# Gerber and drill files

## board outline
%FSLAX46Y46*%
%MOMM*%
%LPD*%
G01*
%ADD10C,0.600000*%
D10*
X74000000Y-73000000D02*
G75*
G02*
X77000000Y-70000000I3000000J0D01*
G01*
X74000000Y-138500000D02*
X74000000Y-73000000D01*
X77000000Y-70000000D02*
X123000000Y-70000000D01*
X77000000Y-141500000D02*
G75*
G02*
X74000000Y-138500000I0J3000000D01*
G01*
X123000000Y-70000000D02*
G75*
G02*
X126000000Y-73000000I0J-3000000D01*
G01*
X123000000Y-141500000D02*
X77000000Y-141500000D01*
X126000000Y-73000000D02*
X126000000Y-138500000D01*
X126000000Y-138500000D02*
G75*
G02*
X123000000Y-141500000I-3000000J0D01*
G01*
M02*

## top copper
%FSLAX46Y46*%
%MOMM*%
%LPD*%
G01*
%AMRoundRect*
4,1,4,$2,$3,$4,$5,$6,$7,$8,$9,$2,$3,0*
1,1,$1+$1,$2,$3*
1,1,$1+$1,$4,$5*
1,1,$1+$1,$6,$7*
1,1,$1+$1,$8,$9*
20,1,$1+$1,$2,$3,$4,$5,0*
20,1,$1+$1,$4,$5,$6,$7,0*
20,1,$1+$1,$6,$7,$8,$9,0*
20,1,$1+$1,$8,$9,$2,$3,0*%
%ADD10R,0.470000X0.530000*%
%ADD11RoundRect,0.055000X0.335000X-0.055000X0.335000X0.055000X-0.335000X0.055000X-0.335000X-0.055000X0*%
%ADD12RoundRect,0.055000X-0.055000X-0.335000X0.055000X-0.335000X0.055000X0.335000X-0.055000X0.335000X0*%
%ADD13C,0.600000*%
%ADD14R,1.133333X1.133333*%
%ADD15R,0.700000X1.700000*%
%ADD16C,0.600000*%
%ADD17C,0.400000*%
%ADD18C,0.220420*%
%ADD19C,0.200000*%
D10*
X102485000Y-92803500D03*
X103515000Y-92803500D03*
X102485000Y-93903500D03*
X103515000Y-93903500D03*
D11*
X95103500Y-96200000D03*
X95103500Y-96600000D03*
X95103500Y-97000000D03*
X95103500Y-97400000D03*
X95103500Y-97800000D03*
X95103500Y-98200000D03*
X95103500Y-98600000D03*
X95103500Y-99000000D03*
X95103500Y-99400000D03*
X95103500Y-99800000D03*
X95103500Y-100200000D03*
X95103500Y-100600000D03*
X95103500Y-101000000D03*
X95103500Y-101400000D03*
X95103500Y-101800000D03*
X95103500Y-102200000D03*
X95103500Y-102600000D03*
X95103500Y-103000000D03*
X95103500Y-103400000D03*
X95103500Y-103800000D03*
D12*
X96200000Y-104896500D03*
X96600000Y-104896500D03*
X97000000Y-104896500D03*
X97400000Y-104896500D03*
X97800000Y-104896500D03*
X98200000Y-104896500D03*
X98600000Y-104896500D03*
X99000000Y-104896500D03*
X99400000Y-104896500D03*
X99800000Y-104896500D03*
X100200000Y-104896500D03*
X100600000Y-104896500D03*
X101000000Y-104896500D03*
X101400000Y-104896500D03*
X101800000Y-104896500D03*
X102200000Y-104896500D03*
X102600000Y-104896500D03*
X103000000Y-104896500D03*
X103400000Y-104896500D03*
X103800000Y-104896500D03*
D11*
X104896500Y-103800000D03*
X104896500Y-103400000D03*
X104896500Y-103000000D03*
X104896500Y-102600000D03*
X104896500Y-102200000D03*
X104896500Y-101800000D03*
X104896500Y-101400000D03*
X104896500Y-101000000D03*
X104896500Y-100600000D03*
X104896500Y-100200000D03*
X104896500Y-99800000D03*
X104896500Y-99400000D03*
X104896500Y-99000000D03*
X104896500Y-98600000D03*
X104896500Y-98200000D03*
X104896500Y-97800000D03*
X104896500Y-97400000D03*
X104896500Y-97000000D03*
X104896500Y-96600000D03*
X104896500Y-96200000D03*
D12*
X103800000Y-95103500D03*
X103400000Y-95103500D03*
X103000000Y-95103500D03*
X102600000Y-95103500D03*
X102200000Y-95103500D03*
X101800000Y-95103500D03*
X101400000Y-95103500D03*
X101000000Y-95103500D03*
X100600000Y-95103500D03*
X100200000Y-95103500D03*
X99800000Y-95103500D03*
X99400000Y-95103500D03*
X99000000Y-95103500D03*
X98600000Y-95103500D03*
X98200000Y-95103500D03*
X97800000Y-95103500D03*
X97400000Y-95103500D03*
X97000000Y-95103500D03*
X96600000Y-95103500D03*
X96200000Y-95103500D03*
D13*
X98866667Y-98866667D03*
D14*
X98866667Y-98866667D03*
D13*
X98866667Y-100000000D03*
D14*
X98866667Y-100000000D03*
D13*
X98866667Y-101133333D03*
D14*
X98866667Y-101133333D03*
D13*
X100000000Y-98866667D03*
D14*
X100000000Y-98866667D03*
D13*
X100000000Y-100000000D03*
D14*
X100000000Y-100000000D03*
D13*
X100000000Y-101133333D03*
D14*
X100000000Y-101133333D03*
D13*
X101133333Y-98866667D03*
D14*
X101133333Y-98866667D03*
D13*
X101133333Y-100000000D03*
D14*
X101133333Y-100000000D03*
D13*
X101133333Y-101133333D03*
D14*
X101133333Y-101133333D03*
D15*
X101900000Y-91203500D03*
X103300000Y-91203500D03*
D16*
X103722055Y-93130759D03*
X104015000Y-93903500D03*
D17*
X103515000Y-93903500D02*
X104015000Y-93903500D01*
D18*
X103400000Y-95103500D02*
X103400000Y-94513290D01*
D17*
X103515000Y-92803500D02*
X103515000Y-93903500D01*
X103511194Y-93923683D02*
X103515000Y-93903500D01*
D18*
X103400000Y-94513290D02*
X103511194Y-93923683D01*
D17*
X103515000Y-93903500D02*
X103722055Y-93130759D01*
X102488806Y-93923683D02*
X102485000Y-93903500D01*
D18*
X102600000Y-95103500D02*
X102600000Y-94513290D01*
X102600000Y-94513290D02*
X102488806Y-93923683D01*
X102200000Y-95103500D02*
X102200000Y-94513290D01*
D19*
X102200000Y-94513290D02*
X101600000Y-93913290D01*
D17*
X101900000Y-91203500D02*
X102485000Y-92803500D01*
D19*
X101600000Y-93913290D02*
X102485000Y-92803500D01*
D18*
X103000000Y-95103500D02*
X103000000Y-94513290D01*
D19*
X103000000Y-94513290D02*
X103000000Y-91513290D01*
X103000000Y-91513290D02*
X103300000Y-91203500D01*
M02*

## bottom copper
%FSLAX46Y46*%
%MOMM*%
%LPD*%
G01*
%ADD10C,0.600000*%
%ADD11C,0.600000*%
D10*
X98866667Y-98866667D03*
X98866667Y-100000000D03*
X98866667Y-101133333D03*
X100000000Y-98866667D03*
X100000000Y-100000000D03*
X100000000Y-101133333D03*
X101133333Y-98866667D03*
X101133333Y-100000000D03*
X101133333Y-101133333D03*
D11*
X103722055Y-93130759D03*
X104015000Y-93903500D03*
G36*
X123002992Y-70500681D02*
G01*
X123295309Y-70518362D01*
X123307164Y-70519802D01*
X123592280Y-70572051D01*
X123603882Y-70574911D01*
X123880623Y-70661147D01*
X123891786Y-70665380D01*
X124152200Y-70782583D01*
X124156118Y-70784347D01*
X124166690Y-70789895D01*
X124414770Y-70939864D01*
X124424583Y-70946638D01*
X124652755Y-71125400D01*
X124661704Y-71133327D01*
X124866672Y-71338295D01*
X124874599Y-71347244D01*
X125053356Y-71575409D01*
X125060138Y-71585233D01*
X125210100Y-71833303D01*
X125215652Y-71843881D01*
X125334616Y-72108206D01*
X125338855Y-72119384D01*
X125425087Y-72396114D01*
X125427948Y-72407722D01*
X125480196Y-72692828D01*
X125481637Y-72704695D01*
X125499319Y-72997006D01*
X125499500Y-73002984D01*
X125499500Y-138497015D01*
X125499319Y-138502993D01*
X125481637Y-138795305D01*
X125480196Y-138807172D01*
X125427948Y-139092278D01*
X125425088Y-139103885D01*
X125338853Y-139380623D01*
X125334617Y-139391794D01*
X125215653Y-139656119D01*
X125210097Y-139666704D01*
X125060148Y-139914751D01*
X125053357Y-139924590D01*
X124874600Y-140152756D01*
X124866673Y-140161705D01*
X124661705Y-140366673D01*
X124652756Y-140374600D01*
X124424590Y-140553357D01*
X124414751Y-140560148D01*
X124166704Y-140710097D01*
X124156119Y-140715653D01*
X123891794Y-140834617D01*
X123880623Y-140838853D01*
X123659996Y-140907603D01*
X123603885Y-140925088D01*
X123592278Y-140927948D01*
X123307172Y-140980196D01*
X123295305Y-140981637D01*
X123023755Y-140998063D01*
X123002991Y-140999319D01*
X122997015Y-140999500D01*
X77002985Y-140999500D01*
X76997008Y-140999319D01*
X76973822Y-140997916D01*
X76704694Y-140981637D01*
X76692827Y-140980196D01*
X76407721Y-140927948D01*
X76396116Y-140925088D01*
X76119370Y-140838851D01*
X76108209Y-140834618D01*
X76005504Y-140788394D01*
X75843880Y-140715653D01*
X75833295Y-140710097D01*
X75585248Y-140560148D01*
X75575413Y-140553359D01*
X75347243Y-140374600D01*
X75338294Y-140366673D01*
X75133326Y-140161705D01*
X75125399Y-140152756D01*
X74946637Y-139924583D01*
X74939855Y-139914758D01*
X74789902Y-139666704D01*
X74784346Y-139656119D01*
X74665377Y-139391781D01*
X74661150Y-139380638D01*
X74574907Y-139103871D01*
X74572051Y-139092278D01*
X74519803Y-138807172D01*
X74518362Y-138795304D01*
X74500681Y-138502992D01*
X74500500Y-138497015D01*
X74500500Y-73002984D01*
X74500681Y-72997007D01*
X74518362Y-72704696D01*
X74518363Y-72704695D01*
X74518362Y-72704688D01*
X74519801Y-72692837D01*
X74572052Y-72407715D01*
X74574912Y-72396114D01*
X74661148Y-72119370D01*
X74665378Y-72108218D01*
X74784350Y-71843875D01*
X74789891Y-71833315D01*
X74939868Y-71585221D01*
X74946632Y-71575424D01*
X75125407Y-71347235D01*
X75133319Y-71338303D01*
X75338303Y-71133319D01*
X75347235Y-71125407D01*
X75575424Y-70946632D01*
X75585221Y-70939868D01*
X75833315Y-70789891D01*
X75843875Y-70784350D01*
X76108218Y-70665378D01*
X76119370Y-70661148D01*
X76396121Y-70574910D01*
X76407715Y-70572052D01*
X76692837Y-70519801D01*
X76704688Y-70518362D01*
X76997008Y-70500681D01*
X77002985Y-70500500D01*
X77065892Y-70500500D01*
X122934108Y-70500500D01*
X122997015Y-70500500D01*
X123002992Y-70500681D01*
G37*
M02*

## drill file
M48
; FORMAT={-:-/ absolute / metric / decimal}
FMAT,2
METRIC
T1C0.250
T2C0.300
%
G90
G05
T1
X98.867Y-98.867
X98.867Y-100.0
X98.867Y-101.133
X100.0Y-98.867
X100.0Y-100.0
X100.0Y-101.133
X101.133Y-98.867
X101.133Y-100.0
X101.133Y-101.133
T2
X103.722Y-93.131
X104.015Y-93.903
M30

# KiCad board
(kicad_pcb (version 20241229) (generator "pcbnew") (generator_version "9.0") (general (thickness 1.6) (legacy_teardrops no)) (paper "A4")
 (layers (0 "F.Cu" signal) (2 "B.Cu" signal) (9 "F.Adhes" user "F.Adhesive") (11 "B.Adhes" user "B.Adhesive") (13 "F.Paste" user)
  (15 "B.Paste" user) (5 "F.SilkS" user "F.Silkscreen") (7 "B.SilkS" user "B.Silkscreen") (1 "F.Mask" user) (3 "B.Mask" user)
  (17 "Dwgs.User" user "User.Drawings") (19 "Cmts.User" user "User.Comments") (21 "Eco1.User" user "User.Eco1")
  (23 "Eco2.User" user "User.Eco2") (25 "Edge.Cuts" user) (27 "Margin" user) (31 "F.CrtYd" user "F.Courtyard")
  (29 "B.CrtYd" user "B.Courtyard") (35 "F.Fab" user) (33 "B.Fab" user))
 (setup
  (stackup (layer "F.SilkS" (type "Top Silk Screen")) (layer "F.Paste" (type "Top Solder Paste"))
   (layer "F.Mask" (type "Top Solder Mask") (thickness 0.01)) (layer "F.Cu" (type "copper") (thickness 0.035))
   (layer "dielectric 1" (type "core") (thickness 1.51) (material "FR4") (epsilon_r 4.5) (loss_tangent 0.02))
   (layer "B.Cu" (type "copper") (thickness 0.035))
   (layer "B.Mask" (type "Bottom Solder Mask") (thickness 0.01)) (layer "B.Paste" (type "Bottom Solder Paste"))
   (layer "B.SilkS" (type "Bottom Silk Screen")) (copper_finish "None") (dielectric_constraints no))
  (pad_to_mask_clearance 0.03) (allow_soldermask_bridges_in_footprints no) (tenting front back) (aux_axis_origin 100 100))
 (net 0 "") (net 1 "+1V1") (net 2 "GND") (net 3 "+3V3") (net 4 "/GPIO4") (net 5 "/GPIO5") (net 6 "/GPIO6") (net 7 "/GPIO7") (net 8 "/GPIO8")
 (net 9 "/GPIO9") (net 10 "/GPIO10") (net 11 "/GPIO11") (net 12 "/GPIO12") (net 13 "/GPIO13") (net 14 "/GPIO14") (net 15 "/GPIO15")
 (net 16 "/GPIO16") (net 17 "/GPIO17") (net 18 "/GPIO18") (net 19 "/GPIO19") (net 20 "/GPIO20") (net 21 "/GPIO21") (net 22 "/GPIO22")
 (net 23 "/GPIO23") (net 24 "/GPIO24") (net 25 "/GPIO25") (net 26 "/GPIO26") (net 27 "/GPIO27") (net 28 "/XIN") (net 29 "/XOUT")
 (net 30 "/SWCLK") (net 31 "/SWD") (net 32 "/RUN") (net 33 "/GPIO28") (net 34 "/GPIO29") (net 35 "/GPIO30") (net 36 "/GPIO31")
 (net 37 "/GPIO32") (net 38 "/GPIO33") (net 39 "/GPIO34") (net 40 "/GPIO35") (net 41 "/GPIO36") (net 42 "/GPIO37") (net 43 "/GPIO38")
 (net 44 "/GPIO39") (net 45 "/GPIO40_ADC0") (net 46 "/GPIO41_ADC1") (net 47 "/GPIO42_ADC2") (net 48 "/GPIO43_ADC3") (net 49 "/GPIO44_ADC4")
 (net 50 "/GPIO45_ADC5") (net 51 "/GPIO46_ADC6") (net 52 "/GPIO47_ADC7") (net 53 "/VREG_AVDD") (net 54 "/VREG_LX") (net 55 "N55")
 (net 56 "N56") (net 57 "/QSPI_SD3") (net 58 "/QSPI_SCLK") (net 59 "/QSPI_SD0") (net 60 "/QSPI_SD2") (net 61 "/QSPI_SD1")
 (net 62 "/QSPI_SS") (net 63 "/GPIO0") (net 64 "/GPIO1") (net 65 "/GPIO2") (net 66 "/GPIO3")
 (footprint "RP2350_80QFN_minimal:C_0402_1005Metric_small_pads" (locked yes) (layer "F.Cu") (at 103 92.8035)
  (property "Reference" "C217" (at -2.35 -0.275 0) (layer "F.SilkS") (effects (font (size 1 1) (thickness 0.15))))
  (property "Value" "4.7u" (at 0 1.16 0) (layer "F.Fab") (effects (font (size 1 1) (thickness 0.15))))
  (pad "1" smd rect (at -0.515 0) (size 0.47 0.53) (layers "F.Cu" "F.Mask" "F.Paste") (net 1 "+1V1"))
  (pad "2" smd rect (at 0.515 0) (size 0.47 0.53) (layers "F.Cu" "F.Mask" "F.Paste") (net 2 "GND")))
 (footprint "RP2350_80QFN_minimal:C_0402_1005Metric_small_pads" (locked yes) (layer "F.Cu") (at 103 93.9035)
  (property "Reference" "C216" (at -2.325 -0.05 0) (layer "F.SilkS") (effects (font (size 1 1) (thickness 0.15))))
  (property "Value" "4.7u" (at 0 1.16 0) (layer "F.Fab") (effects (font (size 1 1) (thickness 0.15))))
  (pad "1" smd rect (at -0.515 0) (size 0.47 0.53) (layers "F.Cu" "F.Mask" "F.Paste") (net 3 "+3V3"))
  (pad "2" smd rect (at 0.515 0) (size 0.47 0.53) (layers "F.Cu" "F.Mask" "F.Paste") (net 2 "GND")))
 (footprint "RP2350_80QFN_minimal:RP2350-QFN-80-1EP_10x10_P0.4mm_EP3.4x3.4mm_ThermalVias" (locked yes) (layer "F.Cu") (at 100 100)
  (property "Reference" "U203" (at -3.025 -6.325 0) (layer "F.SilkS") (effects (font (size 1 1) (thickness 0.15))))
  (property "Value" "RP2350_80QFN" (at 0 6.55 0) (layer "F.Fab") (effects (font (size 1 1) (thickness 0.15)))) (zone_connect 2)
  (pad "" smd roundrect (at -0.7 -0.7) (size 1.2 1.2) (layers "F.Paste") (roundrect_rratio 0.2083333333) (zone_connect 2))
  (pad "" smd roundrect (at -0.7 0.7) (size 1.2 1.2) (layers "F.Paste") (roundrect_rratio 0.2083333333) (zone_connect 2))
  (pad "" smd roundrect (at 0.7 -0.7) (size 1.2 1.2) (layers "F.Paste") (roundrect_rratio 0.2083333333) (zone_connect 2))
  (pad "" smd roundrect (at 0.7 0.7) (size 1.2 1.2) (layers "F.Paste") (roundrect_rratio 0.2083333333) (zone_connect 2))
  (pad "1" smd roundrect (at -4.8965 -3.8 90) (size 0.22 0.78) (layers "F.Cu" "F.Mask" "F.Paste") (roundrect_rratio 0.25) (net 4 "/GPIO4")
   (thermal_bridge_angle 45))
  (pad "2" smd roundrect (at -4.8965 -3.4 90) (size 0.22 0.78) (layers "F.Cu" "F.Mask" "F.Paste") (roundrect_rratio 0.25) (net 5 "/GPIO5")
   (thermal_bridge_angle 45))
  (pad "3" smd roundrect (at -4.8965 -3 90) (size 0.22 0.78) (layers "F.Cu" "F.Mask" "F.Paste") (roundrect_rratio 0.25) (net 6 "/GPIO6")
   (thermal_bridge_angle 45))
  (pad "4" smd roundrect (at -4.8965 -2.6 90) (size 0.22 0.78) (layers "F.Cu" "F.Mask" "F.Paste") (roundrect_rratio 0.25) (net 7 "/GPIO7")
   (thermal_bridge_angle 45))
  (pad "5" smd roundrect (at -4.8965 -2.2 90) (size 0.22 0.78) (layers "F.Cu" "F.Mask" "F.Paste") (roundrect_rratio 0.25) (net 3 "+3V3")
   (thermal_bridge_angle 45))
  (pad "6" smd roundrect (at -4.8965 -1.8 90) (size 0.22 0.78) (layers "F.Cu" "F.Mask" "F.Paste") (roundrect_rratio 0.25) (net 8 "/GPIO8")
   (thermal_bridge_angle 45))
  (pad "7" smd roundrect (at -4.8965 -1.4 90) (size 0.22 0.78) (layers "F.Cu" "F.Mask" "F.Paste") (roundrect_rratio 0.25) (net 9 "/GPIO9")
   (thermal_bridge_angle 45))
  (pad "8" smd roundrect (at -4.8965 -1 90) (size 0.22 0.78) (layers "F.Cu" "F.Mask" "F.Paste") (roundrect_rratio 0.25) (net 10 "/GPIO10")
   (thermal_bridge_angle 45))
  (pad "9" smd roundrect (at -4.8965 -0.6 90) (size 0.22 0.78) (layers "F.Cu" "F.Mask" "F.Paste") (roundrect_rratio 0.25) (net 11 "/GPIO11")
   (thermal_bridge_angle 45))
  (pad "10" smd roundrect (at -4.8965 -0.2 90) (size 0.22 0.78) (layers "F.Cu" "F.Mask" "F.Paste") (roundrect_rratio 0.25) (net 1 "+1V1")
   (thermal_bridge_angle 45))
  (pad "11" smd roundrect (at -4.8965 0.2 90) (size 0.22 0.78) (layers "F.Cu" "F.Mask" "F.Paste") (roundrect_rratio 0.25) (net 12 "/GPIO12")
   (thermal_bridge_angle 45))
  (pad "12" smd roundrect (at -4.8965 0.6 90) (size 0.22 0.78) (layers "F.Cu" "F.Mask" "F.Paste") (roundrect_rratio 0.25) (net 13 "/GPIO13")
   (thermal_bridge_angle 45))
  (pad "13" smd roundrect (at -4.8965 1 90) (size 0.22 0.78) (layers "F.Cu" "F.Mask" "F.Paste") (roundrect_rratio 0.25) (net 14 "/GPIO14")
   (thermal_bridge_angle 45))
  (pad "14" smd roundrect (at -4.8965 1.4 90) (size 0.22 0.78) (layers "F.Cu" "F.Mask" "F.Paste") (roundrect_rratio 0.25) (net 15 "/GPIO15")
   (thermal_bridge_angle 45))
  (pad "15" smd roundrect (at -4.8965 1.8 90) (size 0.22 0.78) (layers "F.Cu" "F.Mask" "F.Paste") (roundrect_rratio 0.25) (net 3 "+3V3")
   (thermal_bridge_angle 45))
  (pad "16" smd roundrect (at -4.8965 2.2 90) (size 0.22 0.78) (layers "F.Cu" "F.Mask" "F.Paste") (roundrect_rratio 0.25) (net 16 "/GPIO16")
   (thermal_bridge_angle 45))
  (pad "17" smd roundrect (at -4.8965 2.6 90) (size 0.22 0.78) (layers "F.Cu" "F.Mask" "F.Paste") (roundrect_rratio 0.25) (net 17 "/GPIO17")
   (thermal_bridge_angle 45))
  (pad "18" smd roundrect (at -4.8965 3 90) (size 0.22 0.78) (layers "F.Cu" "F.Mask" "F.Paste") (roundrect_rratio 0.25) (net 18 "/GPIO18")
   (thermal_bridge_angle 45))
  (pad "19" smd roundrect (at -4.8965 3.4 90) (size 0.22 0.78) (layers "F.Cu" "F.Mask" "F.Paste") (roundrect_rratio 0.25) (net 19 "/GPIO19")
   (thermal_bridge_angle 45))
  (pad "20" smd roundrect (at -4.8965 3.8 90) (size 0.22 0.78) (layers "F.Cu" "F.Mask" "F.Paste") (roundrect_rratio 0.25) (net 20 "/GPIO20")
   (thermal_bridge_angle 45))
  (pad "21" smd roundrect (at -3.8 4.8965) (size 0.22 0.78) (layers "F.Cu" "F.Mask" "F.Paste") (roundrect_rratio 0.25) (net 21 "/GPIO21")
   (thermal_bridge_angle 45))
  (pad "22" smd roundrect (at -3.4 4.8965) (size 0.22 0.78) (layers "F.Cu" "F.Mask" "F.Paste") (roundrect_rratio 0.25) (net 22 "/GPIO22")
   (thermal_bridge_angle 45))
  (pad "23" smd roundrect (at -3 4.8965) (size 0.22 0.78) (layers "F.Cu" "F.Mask" "F.Paste") (roundrect_rratio 0.25) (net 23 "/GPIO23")
   (thermal_bridge_angle 45))
  (pad "24" smd roundrect (at -2.6 4.8965) (size 0.22 0.78) (layers "F.Cu" "F.Mask" "F.Paste") (roundrect_rratio 0.25) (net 3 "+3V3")
   (thermal_bridge_angle 45))
  (pad "25" smd roundrect (at -2.2 4.8965) (size 0.22 0.78) (layers "F.Cu" "F.Mask" "F.Paste") (roundrect_rratio 0.25) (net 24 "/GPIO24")
   (thermal_bridge_angle 45))
  (pad "26" smd roundrect (at -1.8 4.8965) (size 0.22 0.78) (layers "F.Cu" "F.Mask" "F.Paste") (roundrect_rratio 0.25) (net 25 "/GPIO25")
   (thermal_bridge_angle 45))
  (pad "27" smd roundrect (at -1.4 4.8965) (size 0.22 0.78) (layers "F.Cu" "F.Mask" "F.Paste") (roundrect_rratio 0.25) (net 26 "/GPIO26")
   (thermal_bridge_angle 45))
  (pad "28" smd roundrect (at -1 4.8965) (size 0.22 0.78) (layers "F.Cu" "F.Mask" "F.Paste") (roundrect_rratio 0.25) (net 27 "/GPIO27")
   (thermal_bridge_angle 45))
  (pad "29" smd roundrect (at -0.6 4.8965) (size 0.22 0.78) (layers "F.Cu" "F.Mask" "F.Paste") (roundrect_rratio 0.25) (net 3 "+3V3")
   (thermal_bridge_angle 45))
  (pad "30" smd roundrect (at -0.2 4.8965) (size 0.22 0.78) (layers "F.Cu" "F.Mask" "F.Paste") (roundrect_rratio 0.25) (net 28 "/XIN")
   (thermal_bridge_angle 45))
  (pad "31" smd roundrect (at 0.2 4.8965) (size 0.22 0.78) (layers "F.Cu" "F.Mask" "F.Paste") (roundrect_rratio 0.25) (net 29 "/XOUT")
   (thermal_bridge_angle 45))
  (pad "32" smd roundrect (at 0.6 4.8965) (size 0.22 0.78) (layers "F.Cu" "F.Mask" "F.Paste") (roundrect_rratio 0.25) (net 1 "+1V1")
   (thermal_bridge_angle 45))
  (pad "33" smd roundrect (at 1 4.8965) (size 0.22 0.78) (layers "F.Cu" "F.Mask" "F.Paste") (roundrect_rratio 0.25) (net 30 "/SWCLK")
   (thermal_bridge_angle 45))
  (pad "34" smd roundrect (at 1.4 4.8965) (size 0.22 0.78) (layers "F.Cu" "F.Mask" "F.Paste") (roundrect_rratio 0.25) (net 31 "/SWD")
   (thermal_bridge_angle 45))
  (pad "35" smd roundrect (at 1.8 4.8965) (size 0.22 0.78) (layers "F.Cu" "F.Mask" "F.Paste") (roundrect_rratio 0.25) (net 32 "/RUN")
   (thermal_bridge_angle 45))
  (pad "36" smd roundrect (at 2.2 4.8965) (size 0.22 0.78) (layers "F.Cu" "F.Mask" "F.Paste") (roundrect_rratio 0.25) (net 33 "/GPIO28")
   (thermal_bridge_angle 45))
  (pad "37" smd roundrect (at 2.6 4.8965) (size 0.22 0.78) (layers "F.Cu" "F.Mask" "F.Paste") (roundrect_rratio 0.25) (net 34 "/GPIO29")
   (thermal_bridge_angle 45))
  (pad "38" smd roundrect (at 3 4.8965) (size 0.22 0.78) (layers "F.Cu" "F.Mask" "F.Paste") (roundrect_rratio 0.25) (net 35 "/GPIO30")
   (thermal_bridge_angle 45))
  (pad "39" smd roundrect (at 3.4 4.8965) (size 0.22 0.78) (layers "F.Cu" "F.Mask" "F.Paste") (roundrect_rratio 0.25) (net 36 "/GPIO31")
   (thermal_bridge_angle 45))
  (pad "40" smd roundrect (at 3.8 4.8965) (size 0.22 0.78) (layers "F.Cu" "F.Mask" "F.Paste") (roundrect_rratio 0.25) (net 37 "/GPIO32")
   (thermal_bridge_angle 45))
  (pad "41" smd roundrect (at 4.8965 3.8 90) (size 0.22 0.78) (layers "F.Cu" "F.Mask" "F.Paste") (roundrect_rratio 0.25) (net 3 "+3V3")
   (thermal_bridge_angle 45))
  (pad "42" smd roundrect (at 4.8965 3.4 90) (size 0.22 0.78) (layers "F.Cu" "F.Mask" "F.Paste") (roundrect_rratio 0.25) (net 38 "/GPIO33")
   (thermal_bridge_angle 45))
  (pad "43" smd roundrect (at 4.8965 3 90) (size 0.22 0.78) (layers "F.Cu" "F.Mask" "F.Paste") (roundrect_rratio 0.25) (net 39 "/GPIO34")
   (thermal_bridge_angle 45))
  (pad "44" smd roundrect (at 4.8965 2.6 90) (size 0.22 0.78) (layers "F.Cu" "F.Mask" "F.Paste") (roundrect_rratio 0.25) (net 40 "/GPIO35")
   (thermal_bridge_angle 45))
  (pad "45" smd roundrect (at 4.8965 2.2 90) (size 0.22 0.78) (layers "F.Cu" "F.Mask" "F.Paste") (roundrect_rratio 0.25) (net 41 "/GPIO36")
   (thermal_bridge_angle 45))
  (pad "46" smd roundrect (at 4.8965 1.8 90) (size 0.22 0.78) (layers "F.Cu" "F.Mask" "F.Paste") (roundrect_rratio 0.25) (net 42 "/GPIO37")
   (thermal_bridge_angle 45))
  (pad "47" smd roundrect (at 4.8965 1.4 90) (size 0.22 0.78) (layers "F.Cu" "F.Mask" "F.Paste") (roundrect_rratio 0.25) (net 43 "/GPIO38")
   (thermal_bridge_angle 45))
  (pad "48" smd roundrect (at 4.8965 1 90) (size 0.22 0.78) (layers "F.Cu" "F.Mask" "F.Paste") (roundrect_rratio 0.25) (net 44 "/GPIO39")
   (thermal_bridge_angle 45))
  (pad "49" smd roundrect (at 4.8965 0.6 90) (size 0.22 0.78) (layers "F.Cu" "F.Mask" "F.Paste") (roundrect_rratio 0.25)
   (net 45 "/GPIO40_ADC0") (thermal_bridge_angle 45))
  (pad "50" smd roundrect (at 4.8965 0.2 90) (size 0.22 0.78) (layers "F.Cu" "F.Mask" "F.Paste") (roundrect_rratio 0.25) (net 3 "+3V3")
   (thermal_bridge_angle 45))
  (pad "51" smd roundrect (at 4.8965 -0.2 90) (size 0.22 0.78) (layers "F.Cu" "F.Mask" "F.Paste") (roundrect_rratio 0.25) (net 1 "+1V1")
   (thermal_bridge_angle 45))
  (pad "52" smd roundrect (at 4.8965 -0.6 90) (size 0.22 0.78) (layers "F.Cu" "F.Mask" "F.Paste") (roundrect_rratio 0.25)
   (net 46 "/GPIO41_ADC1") (thermal_bridge_angle 45))
  (pad "53" smd roundrect (at 4.8965 -1 90) (size 0.22 0.78) (layers "F.Cu" "F.Mask" "F.Paste") (roundrect_rratio 0.25)
   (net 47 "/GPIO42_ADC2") (thermal_bridge_angle 45))
  (pad "54" smd roundrect (at 4.8965 -1.4 90) (size 0.22 0.78) (layers "F.Cu" "F.Mask" "F.Paste") (roundrect_rratio 0.25)
   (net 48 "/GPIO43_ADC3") (thermal_bridge_angle 45))
  (pad "55" smd roundrect (at 4.8965 -1.8 90) (size 0.22 0.78) (layers "F.Cu" "F.Mask" "F.Paste") (roundrect_rratio 0.25)
   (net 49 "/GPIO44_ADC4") (thermal_bridge_angle 45))
  (pad "56" smd roundrect (at 4.8965 -2.2 90) (size 0.22 0.78) (layers "F.Cu" "F.Mask" "F.Paste") (roundrect_rratio 0.25)
   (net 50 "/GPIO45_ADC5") (thermal_bridge_angle 45))
  (pad "57" smd roundrect (at 4.8965 -2.6 90) (size 0.22 0.78) (layers "F.Cu" "F.Mask" "F.Paste") (roundrect_rratio 0.25)
   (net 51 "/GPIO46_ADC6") (thermal_bridge_angle 45))
  (pad "58" smd roundrect (at 4.8965 -3 90) (size 0.22 0.78) (layers "F.Cu" "F.Mask" "F.Paste") (roundrect_rratio 0.25)
   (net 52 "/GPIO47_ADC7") (thermal_bridge_angle 45))
  (pad "59" smd roundrect (at 4.8965 -3.4 90) (size 0.22 0.78) (layers "F.Cu" "F.Mask" "F.Paste") (roundrect_rratio 0.25) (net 3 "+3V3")
   (thermal_bridge_angle 45))
  (pad "60" smd roundrect (at 4.8965 -3.8 90) (size 0.22 0.78) (layers "F.Cu" "F.Mask" "F.Paste") (roundrect_rratio 0.25) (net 3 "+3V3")
   (thermal_bridge_angle 45))
  (pad "61" smd roundrect (at 3.8 -4.8965) (size 0.22 0.78) (layers "F.Cu" "F.Mask" "F.Paste") (roundrect_rratio 0.25) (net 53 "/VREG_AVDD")
   (thermal_bridge_angle 45))
  (pad "62" smd roundrect (at 3.4 -4.8965) (size 0.22 0.78) (layers "F.Cu" "F.Mask" "F.Paste") (roundrect_rratio 0.25) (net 2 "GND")
   (thermal_bridge_angle 45))
  (pad "63" smd roundrect (at 3 -4.8965) (size 0.22 0.78) (layers "F.Cu" "F.Mask" "F.Paste") (roundrect_rratio 0.25) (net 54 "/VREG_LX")
   (thermal_bridge_angle 45))
  (pad "64" smd roundrect (at 2.6 -4.8965) (size 0.22 0.78) (layers "F.Cu" "F.Mask" "F.Paste") (roundrect_rratio 0.25) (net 3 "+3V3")
   (thermal_bridge_angle 45))
  (pad "65" smd roundrect (at 2.2 -4.8965) (size 0.22 0.78) (layers "F.Cu" "F.Mask" "F.Paste") (roundrect_rratio 0.25) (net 1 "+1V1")
   (thermal_bridge_angle 45))
  (pad "66" smd roundrect (at 1.8 -4.8965) (size 0.22 0.78) (layers "F.Cu" "F.Mask" "F.Paste") (roundrect_rratio 0.25) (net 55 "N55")
   (thermal_bridge_angle 45))
  (pad "67" smd roundrect (at 1.4 -4.8965) (size 0.22 0.78) (layers "F.Cu" "F.Mask" "F.Paste") (roundrect_rratio 0.25) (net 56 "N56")
   (thermal_bridge_angle 45))
  (pad "68" smd roundrect (at 1 -4.8965) (size 0.22 0.78) (layers "F.Cu" "F.Mask" "F.Paste") (roundrect_rratio 0.25) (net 3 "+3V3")
   (thermal_bridge_angle 45))
  (pad "69" smd roundrect (at 0.6 -4.8965) (size 0.22 0.78) (layers "F.Cu" "F.Mask" "F.Paste") (roundrect_rratio 0.25) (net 3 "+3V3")
   (thermal_bridge_angle 45))
  (pad "70" smd roundrect (at 0.2 -4.8965) (size 0.22 0.78) (layers "F.Cu" "F.Mask" "F.Paste") (roundrect_rratio 0.25) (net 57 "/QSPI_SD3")
   (thermal_bridge_angle 45))
  (pad "71" smd roundrect (at -0.2 -4.8965) (size 0.22 0.78) (layers "F.Cu" "F.Mask" "F.Paste") (roundrect_rratio 0.25)
   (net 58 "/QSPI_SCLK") (thermal_bridge_angle 45))
  (pad "72" smd roundrect (at -0.6 -4.8965) (size 0.22 0.78) (layers "F.Cu" "F.Mask" "F.Paste") (roundrect_rratio 0.25) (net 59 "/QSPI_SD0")
   (thermal_bridge_angle 45))
  (pad "73" smd roundrect (at -1 -4.8965) (size 0.22 0.78) (layers "F.Cu" "F.Mask" "F.Paste") (roundrect_rratio 0.25) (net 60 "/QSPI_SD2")
   (thermal_bridge_angle 45))
  (pad "74" smd roundrect (at -1.4 -4.8965) (size 0.22 0.78) (layers "F.Cu" "F.Mask" "F.Paste") (roundrect_rratio 0.25) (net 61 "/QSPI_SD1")
   (thermal_bridge_angle 45))
  (pad "75" smd roundrect (at -1.8 -4.8965) (size 0.22 0.78) (layers "F.Cu" "F.Mask" "F.Paste") (roundrect_rratio 0.25) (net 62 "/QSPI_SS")
   (thermal_bridge_angle 45))
  (pad "76" smd roundrect (at -2.2 -4.8965) (size 0.22 0.78) (layers "F.Cu" "F.Mask" "F.Paste") (roundrect_rratio 0.25) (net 3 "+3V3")
   (thermal_bridge_angle 45))
  (pad "77" smd roundrect (at -2.6 -4.8965) (size 0.22 0.78) (layers "F.Cu" "F.Mask" "F.Paste") (roundrect_rratio 0.25) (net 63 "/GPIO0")
   (thermal_bridge_angle 45))
  (pad "78" smd roundrect (at -3 -4.8965) (size 0.22 0.78) (layers "F.Cu" "F.Mask" "F.Paste") (roundrect_rratio 0.25) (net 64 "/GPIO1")
   (thermal_bridge_angle 45))
  (pad "79" smd roundrect (at -3.4 -4.8965) (size 0.22 0.78) (layers "F.Cu" "F.Mask" "F.Paste") (roundrect_rratio 0.25) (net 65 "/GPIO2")
   (thermal_bridge_angle 45))
  (pad "80" smd roundrect (at -3.8 -4.8965) (size 0.22 0.78) (layers "F.Cu" "F.Mask" "F.Paste") (roundrect_rratio 0.25) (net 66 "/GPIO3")
   (thermal_bridge_angle 45))
  (pad "81" thru_hole circle (at -1.133333 -1.133333) (size 0.6 0.6) (drill 0.25) (layers "*.Cu" "*.Mask") (remove_unused_layers no)
   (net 2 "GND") (zone_connect 2))
  (pad "81" smd rect (at -1.133333 -1.133333) (size 1.133333 1.133333) (layers "F.Cu" "F.Mask" "F.Paste") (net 2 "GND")
   (solder_paste_margin -0.5) (thermal_bridge_angle 45))
  (pad "81" thru_hole circle (at -1.133333 0) (size 0.6 0.6) (drill 0.25) (layers "*.Cu" "*.Mask") (remove_unused_layers no) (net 2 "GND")
   (zone_connect 2))
  (pad "81" smd rect (at -1.133333 0) (size 1.133333 1.133333) (layers "F.Cu" "F.Mask" "F.Paste") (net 2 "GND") (solder_paste_margin -0.5)
   (thermal_bridge_angle 45))
  (pad "81" thru_hole circle (at -1.133333 1.133333) (size 0.6 0.6) (drill 0.25) (layers "*.Cu" "*.Mask") (remove_unused_layers no)
   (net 2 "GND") (zone_connect 2))
  (pad "81" smd rect (at -1.133333 1.133333) (size 1.133333 1.133333) (layers "F.Cu" "F.Mask" "F.Paste") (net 2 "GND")
   (solder_paste_margin -0.5) (thermal_bridge_angle 45))
  (pad "81" thru_hole circle (at 0 -1.133333) (size 0.6 0.6) (drill 0.25) (layers "*.Cu" "*.Mask") (remove_unused_layers no) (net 2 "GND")
   (zone_connect 2))
  (pad "81" smd rect (at 0 -1.133333) (size 1.133333 1.133333) (layers "F.Cu" "F.Mask" "F.Paste") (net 2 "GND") (solder_paste_margin -0.5)
   (thermal_bridge_angle 45))
  (pad "81" thru_hole circle (at 0 0) (size 0.6 0.6) (drill 0.25) (layers "*.Cu" "*.Mask") (remove_unused_layers no) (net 2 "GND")
   (zone_connect 2))
  (pad "81" smd rect (at 0 0) (size 1.133333 1.133333) (layers "F.Cu" "F.Mask" "F.Paste") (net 2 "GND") (solder_paste_margin -0.5)
   (thermal_bridge_angle 45))
  (pad "81" thru_hole circle (at 0 1.133333) (size 0.6 0.6) (drill 0.25) (layers "*.Cu" "*.Mask") (remove_unused_layers no) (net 2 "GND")
   (zone_connect 2))
  (pad "81" smd rect (at 0 1.133333) (size 1.133333 1.133333) (layers "F.Cu" "F.Mask" "F.Paste") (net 2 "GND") (solder_paste_margin -0.5)
   (thermal_bridge_angle 45))
  (pad "81" thru_hole circle (at 1.133333 -1.133333) (size 0.6 0.6) (drill 0.25) (layers "*.Cu" "*.Mask") (remove_unused_layers no)
   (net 2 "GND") (zone_connect 2))
  (pad "81" smd rect (at 1.133333 -1.133333) (size 1.133333 1.133333) (layers "F.Cu" "F.Mask" "F.Paste") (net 2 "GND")
   (solder_paste_margin -0.5) (thermal_bridge_angle 45))
  (pad "81" thru_hole circle (at 1.133333 0) (size 0.6 0.6) (drill 0.25) (layers "*.Cu" "*.Mask") (remove_unused_layers no) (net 2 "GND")
   (zone_connect 2))
  (pad "81" smd rect (at 1.133333 0) (size 1.133333 1.133333) (layers "F.Cu" "F.Mask" "F.Paste") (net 2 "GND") (solder_paste_margin -0.5)
   (thermal_bridge_angle 45))
  (pad "81" thru_hole circle (at 1.133333 1.133333) (size 0.6 0.6) (drill 0.25) (layers "*.Cu" "*.Mask") (remove_unused_layers no)
   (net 2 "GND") (zone_connect 2))
  (pad "81" smd rect (at 1.133333 1.133333) (size 1.133333 1.133333) (layers "F.Cu" "F.Mask" "F.Paste") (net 2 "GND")
   (solder_paste_margin -0.5) (thermal_bridge_angle 45)))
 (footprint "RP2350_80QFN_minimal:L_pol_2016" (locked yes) (layer "F.Cu") (at 102.6 91.2035)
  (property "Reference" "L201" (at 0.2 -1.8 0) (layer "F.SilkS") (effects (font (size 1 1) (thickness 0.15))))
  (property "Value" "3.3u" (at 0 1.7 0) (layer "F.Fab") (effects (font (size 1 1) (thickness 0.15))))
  (pad "1" smd rect (at -0.7 0) (size 0.7 1.7) (layers "F.Cu" "F.Mask" "F.Paste") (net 1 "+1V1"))
  (pad "2" smd rect (at 0.7 0) (size 0.7 1.7) (layers "F.Cu" "F.Mask" "F.Paste") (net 54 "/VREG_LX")))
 (gr_arc (start 74 73) (mid 74.87868 70.87868) (end 77 70) (stroke (width 0.6) (type solid)) (layer "Edge.Cuts"))
 (gr_line (start 74 138.5) (end 74 73) (stroke (width 0.6) (type solid)) (layer "Edge.Cuts"))
 (gr_line (start 77 70) (end 123 70) (stroke (width 0.6) (type solid)) (layer "Edge.Cuts"))
 (gr_arc (start 77 141.5) (mid 74.878679 140.621321) (end 74 138.5) (stroke (width 0.6) (type solid)) (layer "Edge.Cuts"))
 (gr_arc (start 123 70) (mid 125.12132 70.87868) (end 126 73) (stroke (width 0.6) (type solid)) (layer "Edge.Cuts"))
 (gr_line (start 123 141.5) (end 77 141.5) (stroke (width 0.6) (type solid)) (layer "Edge.Cuts"))
 (gr_line (start 126 73) (end 126 138.5) (stroke (width 0.6) (type solid)) (layer "Edge.Cuts"))
 (gr_arc (start 126 138.5) (mid 125.121321 140.621321) (end 123 141.5) (stroke (width 0.6) (type solid)) (layer "Edge.Cuts"))
 (segment (start 103.515 93.9035) (end 104.015 93.9035) (width 0.4) (locked yes) (layer "F.Cu") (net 2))
 (segment (start 103.4 95.1035) (end 103.4 94.51329) (width 0.22042) (locked yes) (layer "F.Cu") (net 2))
 (segment (start 103.515 92.8035) (end 103.515 93.9035) (width 0.4) (locked yes) (layer "F.Cu") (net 2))
 (segment (start 103.511194 93.923683) (end 103.515 93.9035) (width 0.4) (locked yes) (layer "F.Cu") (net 2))
 (segment (start 103.4 94.51329) (end 103.511194 93.923683) (width 0.22042) (locked yes) (layer "F.Cu") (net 2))
 (segment (start 103.515 93.9035) (end 103.722055 93.130759) (width 0.4) (locked yes) (layer "F.Cu") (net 2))
 (via (at 103.722055 93.130759) (size 0.6) (drill 0.3) (layers "F.Cu" "B.Cu") (locked yes) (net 2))
 (via (at 104.015 93.9035) (size 0.6) (drill 0.3) (layers "F.Cu" "B.Cu") (locked yes) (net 2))
 (segment (start 102.488806 93.923683) (end 102.485 93.9035) (width 0.4) (locked yes) (layer "F.Cu") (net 3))
 (segment (start 102.6 95.1035) (end 102.6 94.51329) (width 0.22042) (locked yes) (layer "F.Cu") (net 3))
 (segment (start 102.6 94.51329) (end 102.488806 93.923683) (width 0.22042) (locked yes) (layer "F.Cu") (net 3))
 (segment (start 102.2 95.1035) (end 102.2 94.51329) (width 0.22042) (locked yes) (layer "F.Cu") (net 1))
 (segment (start 102.2 94.51329) (end 101.6 93.91329) (width 0.2) (locked yes) (layer "F.Cu") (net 1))
 (segment (start 101.9 91.2035) (end 102.485 92.8035) (width 0.4) (locked yes) (layer "F.Cu") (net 1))
 (segment (start 101.6 93.91329) (end 102.485 92.8035) (width 0.2) (locked yes) (layer "F.Cu") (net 1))
 (segment (start 103 95.1035) (end 103 94.51329) (width 0.22042) (locked yes) (layer "F.Cu") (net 54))
 (segment (start 103 94.51329) (end 103 91.51329) (width 0.2) (locked yes) (layer "F.Cu") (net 54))
 (segment (start 103 91.51329) (end 103.3 91.2035) (width 0.2) (locked yes) (layer "F.Cu") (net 54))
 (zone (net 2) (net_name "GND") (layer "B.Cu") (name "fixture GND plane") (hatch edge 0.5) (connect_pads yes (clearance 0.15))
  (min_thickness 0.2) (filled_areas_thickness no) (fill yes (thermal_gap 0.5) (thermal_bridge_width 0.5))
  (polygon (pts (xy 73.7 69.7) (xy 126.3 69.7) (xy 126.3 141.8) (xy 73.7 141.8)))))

